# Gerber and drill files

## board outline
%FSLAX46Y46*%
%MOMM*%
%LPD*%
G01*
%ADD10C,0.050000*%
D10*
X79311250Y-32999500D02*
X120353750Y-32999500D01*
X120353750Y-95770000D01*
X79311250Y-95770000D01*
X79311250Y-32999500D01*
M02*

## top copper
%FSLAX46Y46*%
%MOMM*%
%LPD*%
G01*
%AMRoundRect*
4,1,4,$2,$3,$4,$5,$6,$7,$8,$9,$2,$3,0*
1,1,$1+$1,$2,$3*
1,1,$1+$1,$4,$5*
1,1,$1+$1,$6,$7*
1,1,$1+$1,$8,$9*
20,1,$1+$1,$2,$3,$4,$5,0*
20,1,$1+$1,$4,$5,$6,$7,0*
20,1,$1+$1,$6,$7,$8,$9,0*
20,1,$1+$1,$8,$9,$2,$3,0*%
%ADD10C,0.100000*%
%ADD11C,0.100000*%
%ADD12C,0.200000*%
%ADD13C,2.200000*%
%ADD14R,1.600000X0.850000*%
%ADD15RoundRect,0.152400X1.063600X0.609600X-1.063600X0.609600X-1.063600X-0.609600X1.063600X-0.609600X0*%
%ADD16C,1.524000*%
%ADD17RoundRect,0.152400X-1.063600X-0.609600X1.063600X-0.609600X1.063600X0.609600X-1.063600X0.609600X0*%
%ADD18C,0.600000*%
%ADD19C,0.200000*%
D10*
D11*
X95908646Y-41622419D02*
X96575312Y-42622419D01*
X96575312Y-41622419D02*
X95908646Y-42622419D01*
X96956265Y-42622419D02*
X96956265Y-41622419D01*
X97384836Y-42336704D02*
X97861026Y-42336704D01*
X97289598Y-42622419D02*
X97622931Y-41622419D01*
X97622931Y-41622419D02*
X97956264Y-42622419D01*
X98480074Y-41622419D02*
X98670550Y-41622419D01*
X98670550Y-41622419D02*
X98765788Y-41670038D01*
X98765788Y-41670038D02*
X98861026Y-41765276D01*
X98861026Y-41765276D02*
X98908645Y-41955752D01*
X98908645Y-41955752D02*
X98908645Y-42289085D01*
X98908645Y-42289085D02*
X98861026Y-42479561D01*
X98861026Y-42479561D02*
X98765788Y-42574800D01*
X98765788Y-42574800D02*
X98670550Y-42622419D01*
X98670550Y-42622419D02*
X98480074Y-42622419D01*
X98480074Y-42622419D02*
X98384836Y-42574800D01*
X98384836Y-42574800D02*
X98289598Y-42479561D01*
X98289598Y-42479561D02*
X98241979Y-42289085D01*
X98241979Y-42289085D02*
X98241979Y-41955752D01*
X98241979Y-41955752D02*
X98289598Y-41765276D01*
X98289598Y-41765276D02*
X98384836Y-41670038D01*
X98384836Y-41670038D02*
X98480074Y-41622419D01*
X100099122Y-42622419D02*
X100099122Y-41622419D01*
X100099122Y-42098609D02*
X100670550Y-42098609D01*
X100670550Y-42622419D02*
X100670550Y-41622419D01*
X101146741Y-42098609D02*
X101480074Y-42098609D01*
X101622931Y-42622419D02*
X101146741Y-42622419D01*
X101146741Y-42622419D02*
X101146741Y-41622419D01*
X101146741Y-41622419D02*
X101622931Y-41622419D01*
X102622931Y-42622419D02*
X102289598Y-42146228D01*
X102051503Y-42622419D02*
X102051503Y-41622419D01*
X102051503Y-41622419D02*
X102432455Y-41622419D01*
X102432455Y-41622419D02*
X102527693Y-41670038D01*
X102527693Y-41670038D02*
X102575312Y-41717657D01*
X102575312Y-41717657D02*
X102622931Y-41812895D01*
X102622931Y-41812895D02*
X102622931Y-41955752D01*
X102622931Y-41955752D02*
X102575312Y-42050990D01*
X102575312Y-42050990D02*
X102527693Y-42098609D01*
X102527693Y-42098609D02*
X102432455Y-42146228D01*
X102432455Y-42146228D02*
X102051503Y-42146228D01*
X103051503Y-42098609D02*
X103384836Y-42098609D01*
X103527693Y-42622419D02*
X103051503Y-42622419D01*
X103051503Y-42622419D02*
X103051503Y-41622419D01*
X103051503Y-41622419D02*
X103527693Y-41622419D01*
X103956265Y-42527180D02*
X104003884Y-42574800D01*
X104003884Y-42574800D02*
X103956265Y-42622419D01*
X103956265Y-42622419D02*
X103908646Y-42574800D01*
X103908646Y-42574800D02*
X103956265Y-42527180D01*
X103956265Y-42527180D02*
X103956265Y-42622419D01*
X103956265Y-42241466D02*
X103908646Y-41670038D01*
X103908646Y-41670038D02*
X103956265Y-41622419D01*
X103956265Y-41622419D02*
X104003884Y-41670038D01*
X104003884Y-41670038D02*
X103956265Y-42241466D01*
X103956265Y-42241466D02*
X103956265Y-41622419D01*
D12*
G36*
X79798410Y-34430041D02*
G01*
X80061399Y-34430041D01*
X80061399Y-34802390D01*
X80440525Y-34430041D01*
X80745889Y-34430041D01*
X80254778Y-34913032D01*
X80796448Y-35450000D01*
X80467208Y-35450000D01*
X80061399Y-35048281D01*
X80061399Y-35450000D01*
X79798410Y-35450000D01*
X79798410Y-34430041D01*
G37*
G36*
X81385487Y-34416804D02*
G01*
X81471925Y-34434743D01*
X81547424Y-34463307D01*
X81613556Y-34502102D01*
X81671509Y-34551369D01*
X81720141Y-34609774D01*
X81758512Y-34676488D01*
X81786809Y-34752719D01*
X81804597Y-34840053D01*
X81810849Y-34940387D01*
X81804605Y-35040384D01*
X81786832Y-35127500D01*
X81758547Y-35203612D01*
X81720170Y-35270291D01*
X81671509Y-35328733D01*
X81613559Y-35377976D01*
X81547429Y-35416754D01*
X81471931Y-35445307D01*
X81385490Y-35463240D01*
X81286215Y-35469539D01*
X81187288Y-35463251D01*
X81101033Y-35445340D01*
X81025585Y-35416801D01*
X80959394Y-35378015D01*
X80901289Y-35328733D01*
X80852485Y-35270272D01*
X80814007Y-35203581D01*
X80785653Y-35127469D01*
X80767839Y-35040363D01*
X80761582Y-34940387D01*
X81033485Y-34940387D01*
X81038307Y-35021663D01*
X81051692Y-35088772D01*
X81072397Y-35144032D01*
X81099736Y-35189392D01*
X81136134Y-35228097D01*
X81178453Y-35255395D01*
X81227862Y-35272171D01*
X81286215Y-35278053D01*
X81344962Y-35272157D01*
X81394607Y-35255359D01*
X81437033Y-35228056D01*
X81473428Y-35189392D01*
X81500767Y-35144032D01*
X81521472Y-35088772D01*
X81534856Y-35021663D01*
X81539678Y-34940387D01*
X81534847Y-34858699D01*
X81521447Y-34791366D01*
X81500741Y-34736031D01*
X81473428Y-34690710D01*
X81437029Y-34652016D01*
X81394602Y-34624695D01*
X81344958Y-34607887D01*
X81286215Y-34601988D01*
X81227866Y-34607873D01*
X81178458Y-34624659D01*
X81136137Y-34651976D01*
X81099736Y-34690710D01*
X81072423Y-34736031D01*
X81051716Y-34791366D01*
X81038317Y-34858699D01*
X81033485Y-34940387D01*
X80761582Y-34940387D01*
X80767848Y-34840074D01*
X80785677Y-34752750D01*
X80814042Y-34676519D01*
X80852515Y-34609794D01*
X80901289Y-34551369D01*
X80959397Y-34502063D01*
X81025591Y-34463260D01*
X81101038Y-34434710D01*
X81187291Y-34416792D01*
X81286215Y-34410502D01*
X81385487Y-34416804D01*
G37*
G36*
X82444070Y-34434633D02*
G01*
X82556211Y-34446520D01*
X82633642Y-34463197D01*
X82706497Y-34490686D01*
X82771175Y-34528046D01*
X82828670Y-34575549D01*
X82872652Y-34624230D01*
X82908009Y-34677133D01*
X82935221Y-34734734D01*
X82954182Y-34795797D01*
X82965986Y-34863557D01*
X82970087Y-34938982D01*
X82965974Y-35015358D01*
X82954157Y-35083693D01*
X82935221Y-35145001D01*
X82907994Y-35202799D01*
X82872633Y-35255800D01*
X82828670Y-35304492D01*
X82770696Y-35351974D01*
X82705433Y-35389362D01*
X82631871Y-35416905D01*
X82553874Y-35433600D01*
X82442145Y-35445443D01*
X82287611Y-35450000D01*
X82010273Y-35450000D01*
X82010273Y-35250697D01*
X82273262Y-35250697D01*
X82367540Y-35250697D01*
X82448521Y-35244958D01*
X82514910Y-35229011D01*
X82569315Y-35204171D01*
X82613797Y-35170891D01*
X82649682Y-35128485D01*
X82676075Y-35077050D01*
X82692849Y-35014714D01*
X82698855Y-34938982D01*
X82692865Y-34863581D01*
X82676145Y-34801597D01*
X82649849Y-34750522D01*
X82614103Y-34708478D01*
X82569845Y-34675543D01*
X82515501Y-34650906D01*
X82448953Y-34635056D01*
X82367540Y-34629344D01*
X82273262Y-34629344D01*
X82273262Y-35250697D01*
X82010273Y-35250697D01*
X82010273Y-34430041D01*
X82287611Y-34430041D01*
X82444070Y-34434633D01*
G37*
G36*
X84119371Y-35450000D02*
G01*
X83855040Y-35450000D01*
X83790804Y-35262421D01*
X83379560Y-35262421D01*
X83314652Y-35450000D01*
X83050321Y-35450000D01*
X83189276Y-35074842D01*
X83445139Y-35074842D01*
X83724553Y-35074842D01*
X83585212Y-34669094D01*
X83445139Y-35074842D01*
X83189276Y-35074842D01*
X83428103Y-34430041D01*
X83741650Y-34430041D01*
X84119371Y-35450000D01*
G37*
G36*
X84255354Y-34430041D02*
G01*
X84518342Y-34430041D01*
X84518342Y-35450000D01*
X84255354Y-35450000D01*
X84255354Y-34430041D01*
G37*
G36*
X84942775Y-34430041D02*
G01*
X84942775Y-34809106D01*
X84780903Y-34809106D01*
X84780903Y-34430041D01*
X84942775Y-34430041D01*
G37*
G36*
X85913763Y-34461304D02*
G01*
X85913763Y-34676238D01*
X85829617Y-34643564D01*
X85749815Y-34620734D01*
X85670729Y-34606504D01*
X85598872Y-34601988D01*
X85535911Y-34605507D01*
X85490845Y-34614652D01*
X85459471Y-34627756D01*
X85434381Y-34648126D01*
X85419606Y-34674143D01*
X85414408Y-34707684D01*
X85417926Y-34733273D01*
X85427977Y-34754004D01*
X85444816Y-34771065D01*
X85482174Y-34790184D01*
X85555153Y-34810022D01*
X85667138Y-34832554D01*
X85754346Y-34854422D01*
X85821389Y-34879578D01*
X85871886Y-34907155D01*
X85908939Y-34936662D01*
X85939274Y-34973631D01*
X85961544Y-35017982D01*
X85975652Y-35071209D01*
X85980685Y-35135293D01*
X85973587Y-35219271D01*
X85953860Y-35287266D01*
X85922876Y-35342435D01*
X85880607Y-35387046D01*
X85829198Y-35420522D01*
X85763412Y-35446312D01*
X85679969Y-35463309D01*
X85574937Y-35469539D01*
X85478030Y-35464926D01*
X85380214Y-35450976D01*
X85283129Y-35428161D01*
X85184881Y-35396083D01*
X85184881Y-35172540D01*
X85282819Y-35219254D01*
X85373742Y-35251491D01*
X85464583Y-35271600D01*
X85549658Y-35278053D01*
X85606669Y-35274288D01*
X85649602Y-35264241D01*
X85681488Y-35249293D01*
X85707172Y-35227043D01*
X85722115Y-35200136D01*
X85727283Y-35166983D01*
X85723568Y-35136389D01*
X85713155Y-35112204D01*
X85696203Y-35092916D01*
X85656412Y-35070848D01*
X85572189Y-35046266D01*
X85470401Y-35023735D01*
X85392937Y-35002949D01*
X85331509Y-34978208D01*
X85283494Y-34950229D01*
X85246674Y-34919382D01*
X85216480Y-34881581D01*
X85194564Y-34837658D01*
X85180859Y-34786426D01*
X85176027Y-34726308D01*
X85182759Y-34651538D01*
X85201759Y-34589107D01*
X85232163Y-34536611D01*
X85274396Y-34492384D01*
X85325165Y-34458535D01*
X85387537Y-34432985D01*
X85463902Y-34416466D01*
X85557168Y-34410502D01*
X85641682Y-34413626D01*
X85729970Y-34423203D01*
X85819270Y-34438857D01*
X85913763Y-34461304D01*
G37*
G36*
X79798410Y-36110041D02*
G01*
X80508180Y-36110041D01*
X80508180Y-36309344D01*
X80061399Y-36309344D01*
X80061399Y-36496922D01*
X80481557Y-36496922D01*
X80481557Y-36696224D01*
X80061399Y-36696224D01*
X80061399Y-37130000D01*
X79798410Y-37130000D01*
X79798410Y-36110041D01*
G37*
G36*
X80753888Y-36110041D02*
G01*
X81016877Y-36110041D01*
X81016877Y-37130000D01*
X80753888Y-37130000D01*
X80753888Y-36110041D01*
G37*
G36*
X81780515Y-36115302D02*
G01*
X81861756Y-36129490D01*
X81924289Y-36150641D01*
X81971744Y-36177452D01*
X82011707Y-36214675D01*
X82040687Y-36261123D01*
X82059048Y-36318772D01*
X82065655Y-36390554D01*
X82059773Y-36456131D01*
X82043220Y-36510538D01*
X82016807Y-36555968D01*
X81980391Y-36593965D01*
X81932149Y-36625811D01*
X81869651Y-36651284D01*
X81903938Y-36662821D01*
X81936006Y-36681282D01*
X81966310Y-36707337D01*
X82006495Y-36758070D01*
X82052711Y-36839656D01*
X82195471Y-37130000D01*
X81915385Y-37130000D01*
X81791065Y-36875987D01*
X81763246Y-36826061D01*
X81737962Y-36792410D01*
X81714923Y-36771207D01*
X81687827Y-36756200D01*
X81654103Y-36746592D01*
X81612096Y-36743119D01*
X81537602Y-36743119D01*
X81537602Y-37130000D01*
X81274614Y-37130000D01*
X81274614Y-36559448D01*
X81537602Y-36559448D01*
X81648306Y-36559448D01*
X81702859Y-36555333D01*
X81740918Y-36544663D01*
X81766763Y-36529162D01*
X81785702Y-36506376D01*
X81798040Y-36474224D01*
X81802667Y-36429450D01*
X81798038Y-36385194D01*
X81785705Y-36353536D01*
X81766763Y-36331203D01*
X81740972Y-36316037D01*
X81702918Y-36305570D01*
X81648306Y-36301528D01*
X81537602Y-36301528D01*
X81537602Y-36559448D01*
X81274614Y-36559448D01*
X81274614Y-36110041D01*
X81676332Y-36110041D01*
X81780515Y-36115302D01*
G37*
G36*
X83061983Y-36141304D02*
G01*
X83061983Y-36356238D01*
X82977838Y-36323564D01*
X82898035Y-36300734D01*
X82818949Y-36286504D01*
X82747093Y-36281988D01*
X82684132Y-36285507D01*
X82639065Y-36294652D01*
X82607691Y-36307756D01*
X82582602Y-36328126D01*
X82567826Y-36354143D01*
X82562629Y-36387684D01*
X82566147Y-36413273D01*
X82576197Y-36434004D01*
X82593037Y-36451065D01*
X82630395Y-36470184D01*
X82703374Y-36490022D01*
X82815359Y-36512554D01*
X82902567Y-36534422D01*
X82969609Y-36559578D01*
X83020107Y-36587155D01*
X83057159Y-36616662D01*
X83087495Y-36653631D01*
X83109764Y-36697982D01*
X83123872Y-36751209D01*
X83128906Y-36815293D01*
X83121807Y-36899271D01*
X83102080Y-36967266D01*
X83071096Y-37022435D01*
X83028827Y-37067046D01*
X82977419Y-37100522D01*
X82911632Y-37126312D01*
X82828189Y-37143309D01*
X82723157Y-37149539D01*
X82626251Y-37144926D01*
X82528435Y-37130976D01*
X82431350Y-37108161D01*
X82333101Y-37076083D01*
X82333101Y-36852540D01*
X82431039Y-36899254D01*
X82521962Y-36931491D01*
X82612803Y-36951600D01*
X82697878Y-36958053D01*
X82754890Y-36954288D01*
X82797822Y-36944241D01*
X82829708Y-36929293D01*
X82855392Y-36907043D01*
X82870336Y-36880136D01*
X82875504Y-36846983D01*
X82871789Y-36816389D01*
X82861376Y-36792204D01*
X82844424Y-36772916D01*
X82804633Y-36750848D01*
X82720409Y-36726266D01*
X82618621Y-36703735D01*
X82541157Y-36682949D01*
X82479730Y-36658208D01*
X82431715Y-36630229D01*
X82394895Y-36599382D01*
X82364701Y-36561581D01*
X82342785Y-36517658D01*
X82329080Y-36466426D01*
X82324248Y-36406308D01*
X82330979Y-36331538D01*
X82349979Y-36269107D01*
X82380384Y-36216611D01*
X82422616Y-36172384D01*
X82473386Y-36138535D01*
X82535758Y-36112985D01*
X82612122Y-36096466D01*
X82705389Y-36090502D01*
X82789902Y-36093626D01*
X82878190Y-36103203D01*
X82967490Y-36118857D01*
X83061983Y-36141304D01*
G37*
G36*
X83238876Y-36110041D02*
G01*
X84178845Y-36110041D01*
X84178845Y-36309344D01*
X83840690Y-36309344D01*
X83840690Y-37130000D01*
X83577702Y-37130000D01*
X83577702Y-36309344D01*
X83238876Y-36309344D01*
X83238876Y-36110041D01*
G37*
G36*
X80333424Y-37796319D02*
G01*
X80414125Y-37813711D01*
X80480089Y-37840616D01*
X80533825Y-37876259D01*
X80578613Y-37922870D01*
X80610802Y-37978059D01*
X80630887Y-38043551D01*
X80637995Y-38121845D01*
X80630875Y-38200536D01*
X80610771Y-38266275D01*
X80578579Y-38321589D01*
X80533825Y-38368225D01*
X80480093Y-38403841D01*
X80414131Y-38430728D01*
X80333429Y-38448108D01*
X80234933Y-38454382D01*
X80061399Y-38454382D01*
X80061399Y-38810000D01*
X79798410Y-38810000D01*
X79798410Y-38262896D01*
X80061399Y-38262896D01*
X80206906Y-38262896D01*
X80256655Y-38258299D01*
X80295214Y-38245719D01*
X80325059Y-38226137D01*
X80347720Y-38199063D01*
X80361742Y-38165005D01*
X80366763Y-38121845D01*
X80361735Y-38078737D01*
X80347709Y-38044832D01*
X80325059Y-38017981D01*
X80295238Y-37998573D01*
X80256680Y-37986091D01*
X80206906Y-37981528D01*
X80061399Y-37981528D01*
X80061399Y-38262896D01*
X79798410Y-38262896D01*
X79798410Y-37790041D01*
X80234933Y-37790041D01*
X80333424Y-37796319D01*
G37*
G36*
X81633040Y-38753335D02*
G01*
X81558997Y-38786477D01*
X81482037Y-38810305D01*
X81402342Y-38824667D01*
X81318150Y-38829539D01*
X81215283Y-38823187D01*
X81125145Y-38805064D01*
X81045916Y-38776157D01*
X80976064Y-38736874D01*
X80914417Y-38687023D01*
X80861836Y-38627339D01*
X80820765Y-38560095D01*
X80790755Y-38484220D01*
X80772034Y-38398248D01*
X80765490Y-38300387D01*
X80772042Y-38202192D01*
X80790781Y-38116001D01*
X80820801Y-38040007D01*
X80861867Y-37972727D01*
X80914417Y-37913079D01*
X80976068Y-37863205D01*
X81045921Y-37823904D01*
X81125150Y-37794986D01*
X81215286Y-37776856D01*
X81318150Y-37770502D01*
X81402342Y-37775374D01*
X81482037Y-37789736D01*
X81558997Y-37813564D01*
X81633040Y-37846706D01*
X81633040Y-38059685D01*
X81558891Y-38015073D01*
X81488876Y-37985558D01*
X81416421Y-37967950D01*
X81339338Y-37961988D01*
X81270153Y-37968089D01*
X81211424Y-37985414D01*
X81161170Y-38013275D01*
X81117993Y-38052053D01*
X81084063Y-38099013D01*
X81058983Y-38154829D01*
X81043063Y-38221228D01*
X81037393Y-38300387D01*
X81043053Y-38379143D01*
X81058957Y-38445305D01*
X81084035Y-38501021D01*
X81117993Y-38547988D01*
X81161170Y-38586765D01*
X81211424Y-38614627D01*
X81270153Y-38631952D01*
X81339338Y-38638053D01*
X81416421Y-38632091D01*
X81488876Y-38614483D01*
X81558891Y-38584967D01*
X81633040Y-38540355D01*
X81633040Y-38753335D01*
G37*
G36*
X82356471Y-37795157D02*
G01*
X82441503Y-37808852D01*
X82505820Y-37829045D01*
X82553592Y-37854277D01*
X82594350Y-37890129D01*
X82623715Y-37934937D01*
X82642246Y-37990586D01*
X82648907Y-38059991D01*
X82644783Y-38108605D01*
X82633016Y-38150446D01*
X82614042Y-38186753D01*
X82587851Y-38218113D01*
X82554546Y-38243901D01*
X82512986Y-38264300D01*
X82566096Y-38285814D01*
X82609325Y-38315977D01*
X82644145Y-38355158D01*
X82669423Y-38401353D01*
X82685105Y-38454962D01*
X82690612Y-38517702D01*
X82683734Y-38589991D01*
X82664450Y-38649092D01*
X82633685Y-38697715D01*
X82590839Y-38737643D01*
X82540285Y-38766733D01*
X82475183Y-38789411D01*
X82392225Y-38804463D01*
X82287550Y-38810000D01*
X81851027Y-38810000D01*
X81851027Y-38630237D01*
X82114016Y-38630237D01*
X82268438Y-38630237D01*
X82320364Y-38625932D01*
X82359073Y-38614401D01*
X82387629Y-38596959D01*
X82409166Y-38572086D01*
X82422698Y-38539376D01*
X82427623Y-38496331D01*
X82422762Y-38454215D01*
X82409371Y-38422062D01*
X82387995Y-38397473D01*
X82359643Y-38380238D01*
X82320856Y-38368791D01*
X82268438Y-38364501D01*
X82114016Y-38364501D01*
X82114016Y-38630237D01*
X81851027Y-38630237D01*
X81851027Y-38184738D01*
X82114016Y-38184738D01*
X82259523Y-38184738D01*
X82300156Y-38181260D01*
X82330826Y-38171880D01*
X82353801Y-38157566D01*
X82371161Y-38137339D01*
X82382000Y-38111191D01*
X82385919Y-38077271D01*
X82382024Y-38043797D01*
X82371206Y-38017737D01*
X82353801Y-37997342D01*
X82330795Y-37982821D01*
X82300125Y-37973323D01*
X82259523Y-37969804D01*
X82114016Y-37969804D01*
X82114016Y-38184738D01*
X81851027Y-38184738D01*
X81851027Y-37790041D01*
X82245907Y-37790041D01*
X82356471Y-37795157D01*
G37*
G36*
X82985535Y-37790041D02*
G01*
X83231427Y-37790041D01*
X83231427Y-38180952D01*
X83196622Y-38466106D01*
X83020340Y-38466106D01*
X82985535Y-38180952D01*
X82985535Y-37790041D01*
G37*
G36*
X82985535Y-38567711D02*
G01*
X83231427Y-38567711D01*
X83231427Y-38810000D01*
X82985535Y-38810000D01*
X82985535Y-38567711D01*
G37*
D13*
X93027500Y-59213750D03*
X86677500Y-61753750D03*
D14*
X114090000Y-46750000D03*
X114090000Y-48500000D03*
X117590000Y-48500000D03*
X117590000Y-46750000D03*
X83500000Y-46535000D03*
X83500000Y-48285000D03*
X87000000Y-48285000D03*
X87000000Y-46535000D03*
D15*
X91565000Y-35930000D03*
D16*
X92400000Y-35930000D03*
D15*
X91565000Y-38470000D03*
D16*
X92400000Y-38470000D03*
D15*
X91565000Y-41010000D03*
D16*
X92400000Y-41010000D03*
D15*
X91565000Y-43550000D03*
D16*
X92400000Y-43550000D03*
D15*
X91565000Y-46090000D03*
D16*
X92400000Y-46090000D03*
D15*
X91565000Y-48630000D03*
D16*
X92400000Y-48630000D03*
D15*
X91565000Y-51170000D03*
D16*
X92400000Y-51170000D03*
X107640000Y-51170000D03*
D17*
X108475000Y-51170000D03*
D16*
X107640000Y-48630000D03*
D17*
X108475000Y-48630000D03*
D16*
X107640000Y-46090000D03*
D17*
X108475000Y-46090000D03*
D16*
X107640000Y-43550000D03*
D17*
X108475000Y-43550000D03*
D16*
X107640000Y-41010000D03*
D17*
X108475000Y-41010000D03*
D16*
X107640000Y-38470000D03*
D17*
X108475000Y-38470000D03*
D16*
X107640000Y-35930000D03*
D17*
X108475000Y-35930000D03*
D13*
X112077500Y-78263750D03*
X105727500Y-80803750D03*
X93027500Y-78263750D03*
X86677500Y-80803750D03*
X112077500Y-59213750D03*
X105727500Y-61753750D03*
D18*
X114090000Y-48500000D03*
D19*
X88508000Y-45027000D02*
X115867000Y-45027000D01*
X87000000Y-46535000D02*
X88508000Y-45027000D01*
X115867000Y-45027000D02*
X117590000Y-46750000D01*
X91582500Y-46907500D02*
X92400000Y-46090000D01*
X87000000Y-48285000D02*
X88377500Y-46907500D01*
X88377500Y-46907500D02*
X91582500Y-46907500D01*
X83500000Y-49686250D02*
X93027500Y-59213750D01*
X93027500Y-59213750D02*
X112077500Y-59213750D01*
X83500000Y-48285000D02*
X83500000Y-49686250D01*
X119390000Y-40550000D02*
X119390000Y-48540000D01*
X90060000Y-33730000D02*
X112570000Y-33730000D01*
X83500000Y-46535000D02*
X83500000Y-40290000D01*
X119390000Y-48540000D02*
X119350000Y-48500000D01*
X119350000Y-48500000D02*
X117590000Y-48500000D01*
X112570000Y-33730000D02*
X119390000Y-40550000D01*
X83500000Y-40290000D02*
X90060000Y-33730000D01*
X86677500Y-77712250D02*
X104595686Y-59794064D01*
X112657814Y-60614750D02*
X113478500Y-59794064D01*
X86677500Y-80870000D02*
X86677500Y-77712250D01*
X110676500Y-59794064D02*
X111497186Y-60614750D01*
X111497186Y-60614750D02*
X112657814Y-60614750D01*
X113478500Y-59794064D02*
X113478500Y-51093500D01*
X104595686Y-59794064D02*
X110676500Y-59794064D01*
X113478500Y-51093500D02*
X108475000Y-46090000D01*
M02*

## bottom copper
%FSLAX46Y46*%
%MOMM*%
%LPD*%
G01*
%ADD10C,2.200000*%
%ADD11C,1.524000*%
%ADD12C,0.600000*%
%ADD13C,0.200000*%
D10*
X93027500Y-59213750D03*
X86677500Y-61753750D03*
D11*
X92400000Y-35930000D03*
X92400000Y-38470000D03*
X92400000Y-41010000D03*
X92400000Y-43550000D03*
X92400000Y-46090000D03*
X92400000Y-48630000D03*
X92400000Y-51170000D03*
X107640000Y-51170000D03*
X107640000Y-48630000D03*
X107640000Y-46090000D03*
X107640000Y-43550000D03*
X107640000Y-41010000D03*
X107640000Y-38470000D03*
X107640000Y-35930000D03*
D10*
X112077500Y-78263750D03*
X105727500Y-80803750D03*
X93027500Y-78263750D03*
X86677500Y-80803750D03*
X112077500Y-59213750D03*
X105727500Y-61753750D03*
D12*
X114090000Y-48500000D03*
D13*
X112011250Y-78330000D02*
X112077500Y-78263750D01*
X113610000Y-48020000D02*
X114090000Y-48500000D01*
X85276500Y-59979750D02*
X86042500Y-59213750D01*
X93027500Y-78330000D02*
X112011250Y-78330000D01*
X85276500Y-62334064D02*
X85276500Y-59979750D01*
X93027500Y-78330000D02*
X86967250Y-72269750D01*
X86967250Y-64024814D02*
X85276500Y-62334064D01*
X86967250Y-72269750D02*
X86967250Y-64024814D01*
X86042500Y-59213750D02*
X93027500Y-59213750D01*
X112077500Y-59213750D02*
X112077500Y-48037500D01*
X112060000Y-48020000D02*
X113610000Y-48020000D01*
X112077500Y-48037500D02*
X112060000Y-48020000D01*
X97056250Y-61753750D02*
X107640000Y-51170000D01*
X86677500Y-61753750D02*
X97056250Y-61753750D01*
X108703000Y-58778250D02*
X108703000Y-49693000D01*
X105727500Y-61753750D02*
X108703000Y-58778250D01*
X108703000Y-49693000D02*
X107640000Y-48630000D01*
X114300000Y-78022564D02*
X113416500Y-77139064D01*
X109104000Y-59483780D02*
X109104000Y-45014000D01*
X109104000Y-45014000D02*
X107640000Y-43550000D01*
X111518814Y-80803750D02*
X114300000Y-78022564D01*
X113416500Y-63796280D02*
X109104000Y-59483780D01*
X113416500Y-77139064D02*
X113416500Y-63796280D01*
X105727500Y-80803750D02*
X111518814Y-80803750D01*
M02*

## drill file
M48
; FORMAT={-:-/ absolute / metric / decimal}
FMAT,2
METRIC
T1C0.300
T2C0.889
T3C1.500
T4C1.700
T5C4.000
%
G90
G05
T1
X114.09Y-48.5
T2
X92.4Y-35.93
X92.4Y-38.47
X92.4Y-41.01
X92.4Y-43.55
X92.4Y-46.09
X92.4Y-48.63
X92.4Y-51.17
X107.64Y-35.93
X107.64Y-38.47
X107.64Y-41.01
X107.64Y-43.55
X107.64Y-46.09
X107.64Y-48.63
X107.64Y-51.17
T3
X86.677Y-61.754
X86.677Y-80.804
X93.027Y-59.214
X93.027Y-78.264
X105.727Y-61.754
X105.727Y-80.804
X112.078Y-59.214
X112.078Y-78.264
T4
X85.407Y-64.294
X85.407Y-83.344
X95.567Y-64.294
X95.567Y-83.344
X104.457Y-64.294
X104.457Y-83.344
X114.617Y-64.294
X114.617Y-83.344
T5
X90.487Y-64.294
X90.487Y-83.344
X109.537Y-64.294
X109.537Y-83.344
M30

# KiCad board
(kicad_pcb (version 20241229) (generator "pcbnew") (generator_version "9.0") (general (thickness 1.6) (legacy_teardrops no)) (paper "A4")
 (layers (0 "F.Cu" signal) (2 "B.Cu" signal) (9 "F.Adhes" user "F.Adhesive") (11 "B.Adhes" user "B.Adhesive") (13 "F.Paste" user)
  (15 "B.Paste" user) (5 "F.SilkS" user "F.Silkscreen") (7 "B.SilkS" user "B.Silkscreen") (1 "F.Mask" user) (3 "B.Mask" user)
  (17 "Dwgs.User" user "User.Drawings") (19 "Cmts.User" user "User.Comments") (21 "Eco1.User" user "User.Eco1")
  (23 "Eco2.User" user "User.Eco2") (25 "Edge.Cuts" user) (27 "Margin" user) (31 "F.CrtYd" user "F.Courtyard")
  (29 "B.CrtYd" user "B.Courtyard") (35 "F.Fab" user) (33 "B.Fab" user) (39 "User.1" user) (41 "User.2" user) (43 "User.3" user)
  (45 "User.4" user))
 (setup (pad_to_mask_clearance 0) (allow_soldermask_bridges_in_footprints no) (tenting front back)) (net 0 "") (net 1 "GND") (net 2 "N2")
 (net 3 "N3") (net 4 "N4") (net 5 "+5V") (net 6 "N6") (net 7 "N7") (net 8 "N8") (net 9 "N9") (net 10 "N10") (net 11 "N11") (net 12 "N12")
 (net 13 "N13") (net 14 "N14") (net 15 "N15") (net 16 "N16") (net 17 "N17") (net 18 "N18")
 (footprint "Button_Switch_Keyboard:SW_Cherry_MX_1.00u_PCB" (layer "F.Cu") (at 93.0275 59.21375)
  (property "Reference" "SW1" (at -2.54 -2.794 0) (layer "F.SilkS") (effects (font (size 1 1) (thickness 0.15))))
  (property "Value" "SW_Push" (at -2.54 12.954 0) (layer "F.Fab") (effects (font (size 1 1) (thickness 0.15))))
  (pad "" np_thru_hole circle (at -7.62 5.08) (size 1.7 1.7) (drill 1.7) (layers "*.Cu" "*.Mask"))
  (pad "" np_thru_hole circle (at -2.54 5.08) (size 4 4) (drill 4) (layers "*.Cu" "*.Mask"))
  (pad "" np_thru_hole circle (at 2.54 5.08) (size 1.7 1.7) (drill 1.7) (layers "*.Cu" "*.Mask"))
  (pad "1" thru_hole circle (at 0 0) (size 2.2 2.2) (drill 1.5) (layers "*.Cu" "*.Mask") (remove_unused_layers no) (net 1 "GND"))
  (pad "2" thru_hole circle (at -6.35 2.54) (size 2.2 2.2) (drill 1.5) (layers "*.Cu" "*.Mask") (remove_unused_layers no) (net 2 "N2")))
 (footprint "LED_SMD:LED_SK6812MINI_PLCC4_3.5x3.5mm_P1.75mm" (layer "F.Cu") (at 115.84 47.625)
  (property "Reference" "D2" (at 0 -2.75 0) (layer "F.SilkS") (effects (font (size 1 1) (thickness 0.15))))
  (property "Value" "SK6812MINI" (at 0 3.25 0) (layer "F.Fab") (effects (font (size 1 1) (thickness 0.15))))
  (pad "1" smd rect (at -1.75 -0.875) (size 1.6 0.85) (layers "F.Cu" "F.Mask" "F.Paste") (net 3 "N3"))
  (pad "2" smd rect (at -1.75 0.875) (size 1.6 0.85) (layers "F.Cu" "F.Mask" "F.Paste") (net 1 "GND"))
  (pad "3" smd rect (at 1.75 0.875) (size 1.6 0.85) (layers "F.Cu" "F.Mask" "F.Paste") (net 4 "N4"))
  (pad "4" smd rect (at 1.75 -0.875) (size 1.6 0.85) (layers "F.Cu" "F.Mask" "F.Paste") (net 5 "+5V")))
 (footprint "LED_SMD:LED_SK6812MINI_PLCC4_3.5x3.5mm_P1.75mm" (layer "F.Cu") (at 85.25 47.41)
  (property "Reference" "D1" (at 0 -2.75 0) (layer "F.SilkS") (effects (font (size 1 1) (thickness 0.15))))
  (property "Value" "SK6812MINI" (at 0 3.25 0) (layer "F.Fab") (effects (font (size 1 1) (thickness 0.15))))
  (pad "1" smd rect (at -1.75 -0.875) (size 1.6 0.85) (layers "F.Cu" "F.Mask" "F.Paste") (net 4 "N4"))
  (pad "2" smd rect (at -1.75 0.875) (size 1.6 0.85) (layers "F.Cu" "F.Mask" "F.Paste") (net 1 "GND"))
  (pad "3" smd rect (at 1.75 0.875) (size 1.6 0.85) (layers "F.Cu" "F.Mask" "F.Paste") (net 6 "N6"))
  (pad "4" smd rect (at 1.75 -0.875) (size 1.6 0.85) (layers "F.Cu" "F.Mask" "F.Paste") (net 5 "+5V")))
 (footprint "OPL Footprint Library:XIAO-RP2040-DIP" (layer "F.Cu") (at 100.02 43.55)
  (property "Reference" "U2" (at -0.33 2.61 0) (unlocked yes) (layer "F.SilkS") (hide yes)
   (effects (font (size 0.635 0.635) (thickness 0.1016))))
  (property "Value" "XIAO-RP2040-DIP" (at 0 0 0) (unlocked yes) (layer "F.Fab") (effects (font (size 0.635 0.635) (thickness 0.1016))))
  (pad "1" smd roundrect (at -8.455 -7.62 180) (size 2.432 1.524) (layers "F.Cu" "F.Mask") (roundrect_rratio 0.1) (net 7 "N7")
   (thermal_bridge_angle 45))
  (pad "1" thru_hole circle (at -7.62 -7.62 180) (size 1.524 1.524) (drill 0.889) (layers "*.Cu" "*.Mask") (remove_unused_layers no)
   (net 7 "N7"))
  (pad "2" smd roundrect (at -8.455 -5.08 180) (size 2.432 1.524) (layers "F.Cu" "F.Mask") (roundrect_rratio 0.1) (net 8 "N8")
   (thermal_bridge_angle 45))
  (pad "2" thru_hole circle (at -7.62 -5.08 180) (size 1.524 1.524) (drill 0.889) (layers "*.Cu" "*.Mask") (remove_unused_layers no)
   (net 8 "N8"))
  (pad "3" smd roundrect (at -8.455 -2.54 180) (size 2.432 1.524) (layers "F.Cu" "F.Mask") (roundrect_rratio 0.1) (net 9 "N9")
   (thermal_bridge_angle 45))
  (pad "3" thru_hole circle (at -7.62 -2.54 180) (size 1.524 1.524) (drill 0.889) (layers "*.Cu" "*.Mask") (remove_unused_layers no)
   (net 9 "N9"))
  (pad "4" smd roundrect (at -8.455 0 180) (size 2.432 1.524) (layers "F.Cu" "F.Mask") (roundrect_rratio 0.1) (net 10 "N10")
   (thermal_bridge_angle 45))
  (pad "4" thru_hole circle (at -7.62 0 180) (size 1.524 1.524) (drill 0.889) (layers "*.Cu" "*.Mask") (remove_unused_layers no)
   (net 10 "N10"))
  (pad "5" smd roundrect (at -8.455 2.54 180) (size 2.432 1.524) (layers "F.Cu" "F.Mask") (roundrect_rratio 0.1) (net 6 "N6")
   (thermal_bridge_angle 45))
  (pad "5" thru_hole circle (at -7.62 2.54 180) (size 1.524 1.524) (drill 0.889) (layers "*.Cu" "*.Mask") (remove_unused_layers no)
   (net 6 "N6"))
  (pad "6" smd roundrect (at -8.455 5.08 180) (size 2.432 1.524) (layers "F.Cu" "F.Mask") (roundrect_rratio 0.1) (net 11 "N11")
   (thermal_bridge_angle 45))
  (pad "6" thru_hole circle (at -7.62 5.08 180) (size 1.524 1.524) (drill 0.889) (layers "*.Cu" "*.Mask") (remove_unused_layers no)
   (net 11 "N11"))
  (pad "7" smd roundrect (at -8.455 7.62 180) (size 2.432 1.524) (layers "F.Cu" "F.Mask") (roundrect_rratio 0.1) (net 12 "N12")
   (thermal_bridge_angle 45))
  (pad "7" thru_hole circle (at -7.62 7.62 180) (size 1.524 1.524) (drill 0.889) (layers "*.Cu" "*.Mask") (remove_unused_layers no)
   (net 12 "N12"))
  (pad "8" thru_hole circle (at 7.62 7.62) (size 1.524 1.524) (drill 0.889) (layers "*.Cu" "*.Mask") (remove_unused_layers no) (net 2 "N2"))
  (pad "8" smd roundrect (at 8.455 7.62) (size 2.432 1.524) (layers "F.Cu" "F.Mask") (roundrect_rratio 0.1) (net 2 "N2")
   (thermal_bridge_angle 45))
  (pad "9" thru_hole circle (at 7.62 5.08) (size 1.524 1.524) (drill 0.889) (layers "*.Cu" "*.Mask") (remove_unused_layers no)
   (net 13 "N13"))
  (pad "9" smd roundrect (at 8.455 5.08) (size 2.432 1.524) (layers "F.Cu" "F.Mask") (roundrect_rratio 0.1) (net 13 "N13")
   (thermal_bridge_angle 45))
  (pad "10" thru_hole circle (at 7.62 2.54) (size 1.524 1.524) (drill 0.889) (layers "*.Cu" "*.Mask") (remove_unused_layers no)
   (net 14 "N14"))
  (pad "10" smd roundrect (at 8.455 2.54) (size 2.432 1.524) (layers "F.Cu" "F.Mask") (roundrect_rratio 0.1) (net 14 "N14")
   (thermal_bridge_angle 45))
  (pad "11" thru_hole circle (at 7.62 0) (size 1.524 1.524) (drill 0.889) (layers "*.Cu" "*.Mask") (remove_unused_layers no) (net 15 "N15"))
  (pad "11" smd roundrect (at 8.455 0) (size 2.432 1.524) (layers "F.Cu" "F.Mask") (roundrect_rratio 0.1) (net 15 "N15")
   (thermal_bridge_angle 45))
  (pad "12" thru_hole circle (at 7.62 -2.54) (size 1.524 1.524) (drill 0.889) (layers "*.Cu" "*.Mask") (remove_unused_layers no)
   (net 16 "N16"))
  (pad "12" smd roundrect (at 8.455 -2.54) (size 2.432 1.524) (layers "F.Cu" "F.Mask") (roundrect_rratio 0.1) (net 16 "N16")
   (thermal_bridge_angle 45))
  (pad "13" thru_hole circle (at 7.62 -5.08) (size 1.524 1.524) (drill 0.889) (layers "*.Cu" "*.Mask") (remove_unused_layers no)
   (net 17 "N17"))
  (pad "13" smd roundrect (at 8.455 -5.08) (size 2.432 1.524) (layers "F.Cu" "F.Mask") (roundrect_rratio 0.1) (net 17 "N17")
   (thermal_bridge_angle 45))
  (pad "14" thru_hole circle (at 7.62 -7.62) (size 1.524 1.524) (drill 0.889) (layers "*.Cu" "*.Mask") (remove_unused_layers no)
   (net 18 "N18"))
  (pad "14" smd roundrect (at 8.455 -7.62) (size 2.432 1.524) (layers "F.Cu" "F.Mask") (roundrect_rratio 0.1) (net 18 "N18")
   (thermal_bridge_angle 45)))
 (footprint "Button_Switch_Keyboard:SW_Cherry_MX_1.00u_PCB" (layer "F.Cu") (at 112.0775 78.26375)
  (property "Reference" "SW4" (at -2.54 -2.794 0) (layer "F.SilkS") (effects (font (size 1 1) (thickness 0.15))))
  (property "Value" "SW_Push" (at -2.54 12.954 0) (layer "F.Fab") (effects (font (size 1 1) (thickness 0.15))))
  (pad "" np_thru_hole circle (at -7.62 5.08) (size 1.7 1.7) (drill 1.7) (layers "*.Cu" "*.Mask"))
  (pad "" np_thru_hole circle (at -2.54 5.08) (size 4 4) (drill 4) (layers "*.Cu" "*.Mask"))
  (pad "" np_thru_hole circle (at 2.54 5.08) (size 1.7 1.7) (drill 1.7) (layers "*.Cu" "*.Mask"))
  (pad "1" thru_hole circle (at 0 0) (size 2.2 2.2) (drill 1.5) (layers "*.Cu" "*.Mask") (remove_unused_layers no) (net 1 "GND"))
  (pad "2" thru_hole circle (at -6.35 2.54) (size 2.2 2.2) (drill 1.5) (layers "*.Cu" "*.Mask") (remove_unused_layers no) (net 15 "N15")))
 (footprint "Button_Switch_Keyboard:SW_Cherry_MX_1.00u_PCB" (layer "F.Cu") (at 93.0275 78.26375)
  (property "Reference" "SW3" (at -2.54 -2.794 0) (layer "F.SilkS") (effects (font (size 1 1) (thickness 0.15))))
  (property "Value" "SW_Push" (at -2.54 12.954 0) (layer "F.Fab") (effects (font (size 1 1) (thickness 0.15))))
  (pad "" np_thru_hole circle (at -7.62 5.08) (size 1.7 1.7) (drill 1.7) (layers "*.Cu" "*.Mask"))
  (pad "" np_thru_hole circle (at -2.54 5.08) (size 4 4) (drill 4) (layers "*.Cu" "*.Mask"))
  (pad "" np_thru_hole circle (at 2.54 5.08) (size 1.7 1.7) (drill 1.7) (layers "*.Cu" "*.Mask"))
  (pad "1" thru_hole circle (at 0 0) (size 2.2 2.2) (drill 1.5) (layers "*.Cu" "*.Mask") (remove_unused_layers no) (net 1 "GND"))
  (pad "2" thru_hole circle (at -6.35 2.54) (size 2.2 2.2) (drill 1.5) (layers "*.Cu" "*.Mask") (remove_unused_layers no) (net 14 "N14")))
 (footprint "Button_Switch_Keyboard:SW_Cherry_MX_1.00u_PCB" (layer "F.Cu") (at 112.0775 59.21375)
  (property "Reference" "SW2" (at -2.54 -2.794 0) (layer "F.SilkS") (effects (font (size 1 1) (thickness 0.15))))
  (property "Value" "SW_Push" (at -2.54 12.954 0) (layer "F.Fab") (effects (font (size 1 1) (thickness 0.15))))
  (pad "" np_thru_hole circle (at -7.62 5.08) (size 1.7 1.7) (drill 1.7) (layers "*.Cu" "*.Mask"))
  (pad "" np_thru_hole circle (at -2.54 5.08) (size 4 4) (drill 4) (layers "*.Cu" "*.Mask"))
  (pad "" np_thru_hole circle (at 2.54 5.08) (size 1.7 1.7) (drill 1.7) (layers "*.Cu" "*.Mask"))
  (pad "1" thru_hole circle (at 0 0) (size 2.2 2.2) (drill 1.5) (layers "*.Cu" "*.Mask") (remove_unused_layers no) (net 1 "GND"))
  (pad "2" thru_hole circle (at -6.35 2.54) (size 2.2 2.2) (drill 1.5) (layers "*.Cu" "*.Mask") (remove_unused_layers no) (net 13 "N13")))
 (gr_rect (start 79.31125 32.9995) (end 120.35375 95.77) (stroke (width 0.05) (type default)) (fill no) (layer "Edge.Cuts"))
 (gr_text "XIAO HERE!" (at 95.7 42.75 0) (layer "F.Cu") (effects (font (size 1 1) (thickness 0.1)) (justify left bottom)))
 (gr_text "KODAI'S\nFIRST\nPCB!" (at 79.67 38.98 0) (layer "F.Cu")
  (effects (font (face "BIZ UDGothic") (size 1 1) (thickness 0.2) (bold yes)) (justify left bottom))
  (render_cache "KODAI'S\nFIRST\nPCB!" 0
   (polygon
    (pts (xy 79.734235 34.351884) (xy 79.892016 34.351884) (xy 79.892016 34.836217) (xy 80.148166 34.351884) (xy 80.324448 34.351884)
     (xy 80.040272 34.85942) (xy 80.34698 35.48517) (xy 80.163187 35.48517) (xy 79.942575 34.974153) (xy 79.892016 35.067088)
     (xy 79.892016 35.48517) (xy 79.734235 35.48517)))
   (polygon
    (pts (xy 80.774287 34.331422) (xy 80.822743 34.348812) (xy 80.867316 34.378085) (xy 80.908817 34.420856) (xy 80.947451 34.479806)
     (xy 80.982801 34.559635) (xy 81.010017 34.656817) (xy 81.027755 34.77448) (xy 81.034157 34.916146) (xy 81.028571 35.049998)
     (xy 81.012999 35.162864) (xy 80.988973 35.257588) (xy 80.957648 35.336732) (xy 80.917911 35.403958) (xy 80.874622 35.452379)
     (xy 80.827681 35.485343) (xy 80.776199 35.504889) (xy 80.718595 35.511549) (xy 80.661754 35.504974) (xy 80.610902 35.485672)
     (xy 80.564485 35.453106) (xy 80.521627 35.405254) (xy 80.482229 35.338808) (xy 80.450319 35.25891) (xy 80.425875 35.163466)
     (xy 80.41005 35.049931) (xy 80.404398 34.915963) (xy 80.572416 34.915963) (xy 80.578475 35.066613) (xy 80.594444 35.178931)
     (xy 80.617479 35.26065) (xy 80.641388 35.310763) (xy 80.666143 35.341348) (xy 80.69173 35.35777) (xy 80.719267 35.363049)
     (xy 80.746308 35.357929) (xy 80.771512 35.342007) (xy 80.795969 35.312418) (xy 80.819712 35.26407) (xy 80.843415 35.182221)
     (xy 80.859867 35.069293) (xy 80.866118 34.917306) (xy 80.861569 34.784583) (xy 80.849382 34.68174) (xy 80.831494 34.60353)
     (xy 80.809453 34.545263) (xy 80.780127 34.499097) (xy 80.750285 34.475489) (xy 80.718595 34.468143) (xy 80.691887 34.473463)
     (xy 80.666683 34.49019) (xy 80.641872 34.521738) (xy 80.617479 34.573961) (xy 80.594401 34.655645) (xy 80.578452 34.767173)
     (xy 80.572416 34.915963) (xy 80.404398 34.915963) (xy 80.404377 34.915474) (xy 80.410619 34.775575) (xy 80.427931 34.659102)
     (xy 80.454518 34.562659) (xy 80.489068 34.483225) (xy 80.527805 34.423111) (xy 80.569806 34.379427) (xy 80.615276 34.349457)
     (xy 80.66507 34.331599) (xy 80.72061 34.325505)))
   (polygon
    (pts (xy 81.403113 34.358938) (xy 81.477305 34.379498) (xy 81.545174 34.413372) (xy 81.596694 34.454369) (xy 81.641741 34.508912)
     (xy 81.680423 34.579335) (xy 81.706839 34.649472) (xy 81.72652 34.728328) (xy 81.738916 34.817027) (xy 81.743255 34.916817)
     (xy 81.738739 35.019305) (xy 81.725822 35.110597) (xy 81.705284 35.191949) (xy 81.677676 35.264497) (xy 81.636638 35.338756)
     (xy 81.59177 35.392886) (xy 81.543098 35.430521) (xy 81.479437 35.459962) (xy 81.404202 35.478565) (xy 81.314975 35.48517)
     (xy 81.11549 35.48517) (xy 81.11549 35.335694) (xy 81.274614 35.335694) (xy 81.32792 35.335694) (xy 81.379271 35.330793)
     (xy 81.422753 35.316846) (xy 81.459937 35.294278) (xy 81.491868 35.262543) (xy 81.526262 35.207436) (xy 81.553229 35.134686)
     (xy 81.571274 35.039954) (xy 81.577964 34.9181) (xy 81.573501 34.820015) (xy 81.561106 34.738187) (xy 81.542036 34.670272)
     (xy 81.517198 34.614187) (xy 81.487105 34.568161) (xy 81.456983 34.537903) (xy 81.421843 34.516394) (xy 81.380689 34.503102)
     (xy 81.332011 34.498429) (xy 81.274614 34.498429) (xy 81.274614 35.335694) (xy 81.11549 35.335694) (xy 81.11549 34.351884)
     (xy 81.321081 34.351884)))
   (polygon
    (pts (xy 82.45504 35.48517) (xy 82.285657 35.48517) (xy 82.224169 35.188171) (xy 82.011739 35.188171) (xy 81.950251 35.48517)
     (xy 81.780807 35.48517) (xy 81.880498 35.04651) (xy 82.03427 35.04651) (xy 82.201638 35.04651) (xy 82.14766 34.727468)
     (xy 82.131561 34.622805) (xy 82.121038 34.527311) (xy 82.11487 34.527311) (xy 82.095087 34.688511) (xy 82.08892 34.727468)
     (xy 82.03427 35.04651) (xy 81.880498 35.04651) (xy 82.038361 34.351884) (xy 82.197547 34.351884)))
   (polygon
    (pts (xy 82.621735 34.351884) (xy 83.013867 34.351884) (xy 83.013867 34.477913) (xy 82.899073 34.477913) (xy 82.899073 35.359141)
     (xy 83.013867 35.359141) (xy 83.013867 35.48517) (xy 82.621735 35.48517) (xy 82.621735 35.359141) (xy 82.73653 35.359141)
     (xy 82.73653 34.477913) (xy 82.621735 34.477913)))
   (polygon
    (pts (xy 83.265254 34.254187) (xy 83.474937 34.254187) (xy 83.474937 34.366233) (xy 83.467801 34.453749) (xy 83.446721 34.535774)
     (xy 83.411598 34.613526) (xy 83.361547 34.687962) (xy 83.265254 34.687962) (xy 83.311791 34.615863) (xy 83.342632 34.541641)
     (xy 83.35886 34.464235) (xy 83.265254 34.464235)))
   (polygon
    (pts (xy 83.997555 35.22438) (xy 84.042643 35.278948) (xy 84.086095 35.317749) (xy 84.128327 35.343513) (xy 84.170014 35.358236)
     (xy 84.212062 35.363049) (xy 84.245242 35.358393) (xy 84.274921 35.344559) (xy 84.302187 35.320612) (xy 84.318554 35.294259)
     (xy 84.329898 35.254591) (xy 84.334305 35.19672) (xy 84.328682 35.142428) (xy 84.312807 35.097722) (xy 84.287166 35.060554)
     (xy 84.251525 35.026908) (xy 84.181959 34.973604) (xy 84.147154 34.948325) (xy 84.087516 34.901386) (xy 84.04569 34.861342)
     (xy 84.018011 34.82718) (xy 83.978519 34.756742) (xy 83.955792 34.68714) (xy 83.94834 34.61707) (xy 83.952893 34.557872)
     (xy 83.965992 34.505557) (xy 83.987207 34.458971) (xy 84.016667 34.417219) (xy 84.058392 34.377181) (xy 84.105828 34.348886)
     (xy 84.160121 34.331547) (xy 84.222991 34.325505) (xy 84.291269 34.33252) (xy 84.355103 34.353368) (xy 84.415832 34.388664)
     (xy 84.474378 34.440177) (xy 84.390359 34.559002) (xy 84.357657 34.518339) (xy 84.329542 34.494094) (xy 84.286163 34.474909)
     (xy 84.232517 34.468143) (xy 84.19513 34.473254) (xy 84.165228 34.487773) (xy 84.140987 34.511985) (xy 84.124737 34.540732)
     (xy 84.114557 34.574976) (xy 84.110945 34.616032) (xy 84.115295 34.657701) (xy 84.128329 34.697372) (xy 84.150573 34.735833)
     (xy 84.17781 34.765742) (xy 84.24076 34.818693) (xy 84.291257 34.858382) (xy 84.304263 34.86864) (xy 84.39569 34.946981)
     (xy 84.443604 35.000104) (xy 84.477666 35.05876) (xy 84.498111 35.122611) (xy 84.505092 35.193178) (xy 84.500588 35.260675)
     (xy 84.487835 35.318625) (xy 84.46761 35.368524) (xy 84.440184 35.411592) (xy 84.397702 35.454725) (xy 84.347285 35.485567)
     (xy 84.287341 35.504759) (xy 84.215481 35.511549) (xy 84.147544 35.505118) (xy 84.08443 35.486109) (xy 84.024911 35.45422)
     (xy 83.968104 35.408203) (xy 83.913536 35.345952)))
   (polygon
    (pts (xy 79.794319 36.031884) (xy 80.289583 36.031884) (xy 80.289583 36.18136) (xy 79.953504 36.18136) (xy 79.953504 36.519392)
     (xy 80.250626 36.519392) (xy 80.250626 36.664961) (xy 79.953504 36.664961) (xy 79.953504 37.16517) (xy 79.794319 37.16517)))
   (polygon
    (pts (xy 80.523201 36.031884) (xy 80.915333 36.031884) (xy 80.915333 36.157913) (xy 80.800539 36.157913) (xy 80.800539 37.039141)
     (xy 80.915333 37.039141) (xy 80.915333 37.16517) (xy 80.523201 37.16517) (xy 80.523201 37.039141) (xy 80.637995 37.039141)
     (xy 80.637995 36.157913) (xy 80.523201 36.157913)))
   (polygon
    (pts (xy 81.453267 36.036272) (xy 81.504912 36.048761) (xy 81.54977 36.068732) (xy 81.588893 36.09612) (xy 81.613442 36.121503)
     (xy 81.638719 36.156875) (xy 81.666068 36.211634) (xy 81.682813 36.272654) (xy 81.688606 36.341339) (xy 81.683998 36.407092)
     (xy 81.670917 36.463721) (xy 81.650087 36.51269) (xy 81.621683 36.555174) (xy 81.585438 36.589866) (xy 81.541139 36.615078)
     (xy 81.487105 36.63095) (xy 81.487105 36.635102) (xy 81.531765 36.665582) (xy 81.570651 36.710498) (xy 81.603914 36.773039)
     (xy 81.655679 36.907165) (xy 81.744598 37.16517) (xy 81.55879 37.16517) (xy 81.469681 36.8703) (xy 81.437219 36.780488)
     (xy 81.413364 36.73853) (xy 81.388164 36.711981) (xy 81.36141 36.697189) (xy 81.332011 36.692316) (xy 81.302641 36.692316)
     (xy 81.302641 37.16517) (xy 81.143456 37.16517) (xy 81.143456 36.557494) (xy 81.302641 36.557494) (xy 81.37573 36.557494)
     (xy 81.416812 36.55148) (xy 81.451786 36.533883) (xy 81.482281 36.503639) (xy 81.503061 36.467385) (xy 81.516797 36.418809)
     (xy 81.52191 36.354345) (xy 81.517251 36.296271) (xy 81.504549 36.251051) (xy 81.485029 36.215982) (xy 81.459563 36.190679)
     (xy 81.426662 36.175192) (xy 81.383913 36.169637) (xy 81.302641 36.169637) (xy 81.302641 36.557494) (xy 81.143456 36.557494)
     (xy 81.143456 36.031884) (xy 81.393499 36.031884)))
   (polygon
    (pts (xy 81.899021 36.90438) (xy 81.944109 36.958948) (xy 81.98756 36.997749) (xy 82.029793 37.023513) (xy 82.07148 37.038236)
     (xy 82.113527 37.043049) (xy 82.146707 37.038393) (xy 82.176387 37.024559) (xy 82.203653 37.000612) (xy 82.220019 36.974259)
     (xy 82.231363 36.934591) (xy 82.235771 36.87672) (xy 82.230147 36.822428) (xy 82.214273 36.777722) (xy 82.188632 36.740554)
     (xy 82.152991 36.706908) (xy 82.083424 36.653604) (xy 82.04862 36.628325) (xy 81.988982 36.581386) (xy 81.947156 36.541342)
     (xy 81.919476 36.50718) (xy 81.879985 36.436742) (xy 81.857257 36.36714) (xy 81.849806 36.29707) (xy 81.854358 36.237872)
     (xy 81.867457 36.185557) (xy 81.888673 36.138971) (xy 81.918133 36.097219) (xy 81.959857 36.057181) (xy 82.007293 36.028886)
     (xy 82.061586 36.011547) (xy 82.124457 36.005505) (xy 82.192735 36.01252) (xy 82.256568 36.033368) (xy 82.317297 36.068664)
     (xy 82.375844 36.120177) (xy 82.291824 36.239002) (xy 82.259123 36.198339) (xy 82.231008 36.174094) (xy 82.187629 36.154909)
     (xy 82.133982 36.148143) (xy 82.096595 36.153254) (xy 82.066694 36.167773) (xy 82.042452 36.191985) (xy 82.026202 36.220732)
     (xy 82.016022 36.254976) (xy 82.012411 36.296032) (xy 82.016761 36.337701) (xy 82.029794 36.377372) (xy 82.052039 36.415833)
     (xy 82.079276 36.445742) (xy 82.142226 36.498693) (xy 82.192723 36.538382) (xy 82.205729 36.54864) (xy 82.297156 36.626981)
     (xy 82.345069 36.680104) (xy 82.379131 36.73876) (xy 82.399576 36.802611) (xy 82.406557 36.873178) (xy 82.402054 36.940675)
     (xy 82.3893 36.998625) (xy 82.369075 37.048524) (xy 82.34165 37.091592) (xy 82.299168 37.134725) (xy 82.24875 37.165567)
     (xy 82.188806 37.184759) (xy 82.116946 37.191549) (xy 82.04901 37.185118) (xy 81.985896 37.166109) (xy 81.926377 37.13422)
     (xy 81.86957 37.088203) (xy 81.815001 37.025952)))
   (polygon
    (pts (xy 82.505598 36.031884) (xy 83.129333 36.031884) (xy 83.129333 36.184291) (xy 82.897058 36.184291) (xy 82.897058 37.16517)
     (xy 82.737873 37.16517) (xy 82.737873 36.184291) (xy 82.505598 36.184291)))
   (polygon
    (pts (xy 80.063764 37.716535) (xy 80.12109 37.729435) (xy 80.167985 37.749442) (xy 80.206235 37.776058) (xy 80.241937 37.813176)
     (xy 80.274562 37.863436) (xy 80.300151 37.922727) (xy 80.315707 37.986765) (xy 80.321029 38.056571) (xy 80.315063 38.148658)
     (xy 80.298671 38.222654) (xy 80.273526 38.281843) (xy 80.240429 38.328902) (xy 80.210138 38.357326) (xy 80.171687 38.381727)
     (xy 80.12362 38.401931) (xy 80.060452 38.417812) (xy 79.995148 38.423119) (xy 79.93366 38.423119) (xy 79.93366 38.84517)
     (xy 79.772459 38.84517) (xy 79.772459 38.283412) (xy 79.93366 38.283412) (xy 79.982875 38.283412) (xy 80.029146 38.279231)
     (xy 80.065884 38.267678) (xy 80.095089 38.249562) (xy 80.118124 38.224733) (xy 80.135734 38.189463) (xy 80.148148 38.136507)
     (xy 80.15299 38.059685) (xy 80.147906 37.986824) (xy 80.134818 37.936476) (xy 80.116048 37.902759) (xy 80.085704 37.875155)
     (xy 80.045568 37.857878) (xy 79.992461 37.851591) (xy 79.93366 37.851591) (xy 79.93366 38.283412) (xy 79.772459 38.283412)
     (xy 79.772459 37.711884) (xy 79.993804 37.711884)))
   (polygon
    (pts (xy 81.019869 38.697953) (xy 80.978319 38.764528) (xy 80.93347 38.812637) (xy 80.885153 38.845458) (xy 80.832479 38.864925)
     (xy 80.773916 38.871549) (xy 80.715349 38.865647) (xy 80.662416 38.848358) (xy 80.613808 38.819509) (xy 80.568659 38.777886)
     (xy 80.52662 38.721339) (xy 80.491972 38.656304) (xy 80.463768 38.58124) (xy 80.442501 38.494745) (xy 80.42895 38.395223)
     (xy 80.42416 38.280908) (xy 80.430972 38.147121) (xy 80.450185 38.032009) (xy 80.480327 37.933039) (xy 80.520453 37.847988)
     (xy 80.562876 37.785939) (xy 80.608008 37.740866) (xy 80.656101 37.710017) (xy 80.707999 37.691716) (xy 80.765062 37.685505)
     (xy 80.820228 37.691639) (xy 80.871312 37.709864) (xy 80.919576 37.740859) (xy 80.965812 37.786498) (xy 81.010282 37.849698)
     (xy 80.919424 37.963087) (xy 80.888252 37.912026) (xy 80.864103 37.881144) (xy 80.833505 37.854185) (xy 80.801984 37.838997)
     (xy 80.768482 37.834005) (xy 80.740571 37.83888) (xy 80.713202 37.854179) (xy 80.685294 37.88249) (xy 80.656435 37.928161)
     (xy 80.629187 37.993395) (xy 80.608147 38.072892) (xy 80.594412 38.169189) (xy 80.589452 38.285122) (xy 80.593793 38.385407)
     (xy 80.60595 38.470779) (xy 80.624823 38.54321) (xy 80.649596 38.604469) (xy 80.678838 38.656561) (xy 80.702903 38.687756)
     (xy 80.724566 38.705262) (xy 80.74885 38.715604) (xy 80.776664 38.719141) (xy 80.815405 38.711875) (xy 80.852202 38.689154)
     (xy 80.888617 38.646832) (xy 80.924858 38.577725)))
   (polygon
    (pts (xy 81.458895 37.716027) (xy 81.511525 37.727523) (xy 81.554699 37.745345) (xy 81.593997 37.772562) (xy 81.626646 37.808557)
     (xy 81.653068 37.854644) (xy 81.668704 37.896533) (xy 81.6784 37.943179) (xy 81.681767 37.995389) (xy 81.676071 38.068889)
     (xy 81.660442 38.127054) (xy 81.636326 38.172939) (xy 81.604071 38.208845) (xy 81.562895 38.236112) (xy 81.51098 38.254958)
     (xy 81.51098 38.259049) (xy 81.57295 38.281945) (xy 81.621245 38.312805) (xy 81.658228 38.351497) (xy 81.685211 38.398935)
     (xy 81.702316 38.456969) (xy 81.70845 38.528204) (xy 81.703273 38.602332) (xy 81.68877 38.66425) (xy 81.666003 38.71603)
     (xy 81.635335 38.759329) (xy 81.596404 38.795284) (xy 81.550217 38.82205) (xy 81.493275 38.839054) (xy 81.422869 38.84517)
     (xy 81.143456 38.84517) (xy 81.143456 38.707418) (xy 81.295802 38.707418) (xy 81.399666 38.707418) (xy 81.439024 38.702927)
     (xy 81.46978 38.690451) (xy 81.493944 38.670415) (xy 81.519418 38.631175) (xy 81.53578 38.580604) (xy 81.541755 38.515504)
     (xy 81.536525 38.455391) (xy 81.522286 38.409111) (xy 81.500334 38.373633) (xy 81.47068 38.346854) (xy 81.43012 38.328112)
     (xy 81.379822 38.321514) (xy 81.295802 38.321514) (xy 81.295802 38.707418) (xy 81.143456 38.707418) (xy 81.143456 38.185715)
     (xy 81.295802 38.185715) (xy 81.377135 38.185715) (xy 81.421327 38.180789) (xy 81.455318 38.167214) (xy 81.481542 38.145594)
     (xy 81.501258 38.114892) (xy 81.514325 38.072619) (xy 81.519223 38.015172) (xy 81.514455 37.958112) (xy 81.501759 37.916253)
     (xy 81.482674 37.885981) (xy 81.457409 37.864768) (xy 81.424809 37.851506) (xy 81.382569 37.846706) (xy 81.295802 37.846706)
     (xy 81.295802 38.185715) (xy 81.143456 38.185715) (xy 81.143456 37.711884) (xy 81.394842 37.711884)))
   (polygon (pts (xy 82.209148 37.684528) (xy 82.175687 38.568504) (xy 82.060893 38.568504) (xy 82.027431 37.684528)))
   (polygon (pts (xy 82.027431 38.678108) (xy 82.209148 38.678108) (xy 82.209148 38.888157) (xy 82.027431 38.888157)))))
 (segment (start 88.508 45.027) (end 115.867 45.027) (width 0.2) (layer "F.Cu") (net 5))
 (segment (start 87 46.535) (end 88.508 45.027) (width 0.2) (layer "F.Cu") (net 5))
 (segment (start 115.867 45.027) (end 117.59 46.75) (width 0.2) (layer "F.Cu") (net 5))
 (segment (start 91.5825 46.9075) (end 92.4 46.09) (width 0.2) (layer "F.Cu") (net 6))
 (segment (start 87 48.285) (end 88.3775 46.9075) (width 0.2) (layer "F.Cu") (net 6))
 (segment (start 88.3775 46.9075) (end 91.5825 46.9075) (width 0.2) (layer "F.Cu") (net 6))
 (segment (start 83.5 49.68625) (end 93.0275 59.21375) (width 0.2) (layer "F.Cu") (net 1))
 (segment (start 93.0275 59.21375) (end 112.0775 59.21375) (width 0.2) (layer "F.Cu") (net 1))
 (segment (start 83.5 48.285) (end 83.5 49.68625) (width 0.2) (layer "F.Cu") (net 1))
 (via (at 114.09 48.5) (size 0.6) (drill 0.3) (layers "F.Cu" "B.Cu") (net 1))
 (segment (start 112.01125 78.33) (end 112.0775 78.26375) (width 0.2) (layer "B.Cu") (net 1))
 (segment (start 113.61 48.02) (end 114.09 48.5) (width 0.2) (layer "B.Cu") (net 1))
 (segment (start 85.2765 59.97975) (end 86.0425 59.21375) (width 0.2) (layer "B.Cu") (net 1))
 (segment (start 93.0275 78.33) (end 112.01125 78.33) (width 0.2) (layer "B.Cu") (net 1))
 (segment (start 85.2765 62.334064) (end 85.2765 59.97975) (width 0.2) (layer "B.Cu") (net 1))
 (segment (start 93.0275 78.33) (end 86.96725 72.26975) (width 0.2) (layer "B.Cu") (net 1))
 (segment (start 86.96725 64.024814) (end 85.2765 62.334064) (width 0.2) (layer "B.Cu") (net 1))
 (segment (start 86.96725 72.26975) (end 86.96725 64.024814) (width 0.2) (layer "B.Cu") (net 1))
 (segment (start 86.0425 59.21375) (end 93.0275 59.21375) (width 0.2) (layer "B.Cu") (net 1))
 (segment (start 112.0775 59.21375) (end 112.0775 48.0375) (width 0.2) (layer "B.Cu") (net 1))
 (segment (start 112.06 48.02) (end 113.61 48.02) (width 0.2) (layer "B.Cu") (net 1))
 (segment (start 112.0775 48.0375) (end 112.06 48.02) (width 0.2) (layer "B.Cu") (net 1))
 (segment (start 119.39 40.55) (end 119.39 48.54) (width 0.2) (layer "F.Cu") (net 4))
 (segment (start 90.06 33.73) (end 112.57 33.73) (width 0.2) (layer "F.Cu") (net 4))
 (segment (start 83.5 46.535) (end 83.5 40.29) (width 0.2) (layer "F.Cu") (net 4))
 (segment (start 119.39 48.54) (end 119.35 48.5) (width 0.2) (layer "F.Cu") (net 4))
 (segment (start 119.35 48.5) (end 117.59 48.5) (width 0.2) (layer "F.Cu") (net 4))
 (segment (start 112.57 33.73) (end 119.39 40.55) (width 0.2) (layer "F.Cu") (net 4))
 (segment (start 83.5 40.29) (end 90.06 33.73) (width 0.2) (layer "F.Cu") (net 4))
 (segment (start 97.05625 61.75375) (end 107.64 51.17) (width 0.2) (layer "B.Cu") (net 2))
 (segment (start 86.6775 61.75375) (end 97.05625 61.75375) (width 0.2) (layer "B.Cu") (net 2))
 (segment (start 108.703 58.77825) (end 108.703 49.693) (width 0.2) (layer "B.Cu") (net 13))
 (segment (start 105.7275 61.75375) (end 108.703 58.77825) (width 0.2) (layer "B.Cu") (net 13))
 (segment (start 108.703 49.693) (end 107.64 48.63) (width 0.2) (layer "B.Cu") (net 13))
 (segment (start 86.6775 77.71225) (end 104.595686 59.794064) (width 0.2) (layer "F.Cu") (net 14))
 (segment (start 112.657814 60.61475) (end 113.4785 59.794064) (width 0.2) (layer "F.Cu") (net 14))
 (segment (start 86.6775 80.87) (end 86.6775 77.71225) (width 0.2) (layer "F.Cu") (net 14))
 (segment (start 110.6765 59.794064) (end 111.497186 60.61475) (width 0.2) (layer "F.Cu") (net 14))
 (segment (start 111.497186 60.61475) (end 112.657814 60.61475) (width 0.2) (layer "F.Cu") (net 14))
 (segment (start 113.4785 59.794064) (end 113.4785 51.0935) (width 0.2) (layer "F.Cu") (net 14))
 (segment (start 104.595686 59.794064) (end 110.6765 59.794064) (width 0.2) (layer "F.Cu") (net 14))
 (segment (start 113.4785 51.0935) (end 108.475 46.09) (width 0.2) (layer "F.Cu") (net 14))
 (segment (start 114.3 78.022564) (end 113.4165 77.139064) (width 0.2) (layer "B.Cu") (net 15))
 (segment (start 109.104 59.48378) (end 109.104 45.014) (width 0.2) (layer "B.Cu") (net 15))
 (segment (start 109.104 45.014) (end 107.64 43.55) (width 0.2) (layer "B.Cu") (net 15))
 (segment (start 111.518814 80.80375) (end 114.3 78.022564) (width 0.2) (layer "B.Cu") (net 15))
 (segment (start 113.4165 63.79628) (end 109.104 59.48378) (width 0.2) (layer "B.Cu") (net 15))
 (segment (start 113.4165 77.139064) (end 113.4165 63.79628) (width 0.2) (layer "B.Cu") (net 15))
 (segment (start 105.7275 80.80375) (end 111.518814 80.80375) (width 0.2) (layer "B.Cu") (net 15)))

